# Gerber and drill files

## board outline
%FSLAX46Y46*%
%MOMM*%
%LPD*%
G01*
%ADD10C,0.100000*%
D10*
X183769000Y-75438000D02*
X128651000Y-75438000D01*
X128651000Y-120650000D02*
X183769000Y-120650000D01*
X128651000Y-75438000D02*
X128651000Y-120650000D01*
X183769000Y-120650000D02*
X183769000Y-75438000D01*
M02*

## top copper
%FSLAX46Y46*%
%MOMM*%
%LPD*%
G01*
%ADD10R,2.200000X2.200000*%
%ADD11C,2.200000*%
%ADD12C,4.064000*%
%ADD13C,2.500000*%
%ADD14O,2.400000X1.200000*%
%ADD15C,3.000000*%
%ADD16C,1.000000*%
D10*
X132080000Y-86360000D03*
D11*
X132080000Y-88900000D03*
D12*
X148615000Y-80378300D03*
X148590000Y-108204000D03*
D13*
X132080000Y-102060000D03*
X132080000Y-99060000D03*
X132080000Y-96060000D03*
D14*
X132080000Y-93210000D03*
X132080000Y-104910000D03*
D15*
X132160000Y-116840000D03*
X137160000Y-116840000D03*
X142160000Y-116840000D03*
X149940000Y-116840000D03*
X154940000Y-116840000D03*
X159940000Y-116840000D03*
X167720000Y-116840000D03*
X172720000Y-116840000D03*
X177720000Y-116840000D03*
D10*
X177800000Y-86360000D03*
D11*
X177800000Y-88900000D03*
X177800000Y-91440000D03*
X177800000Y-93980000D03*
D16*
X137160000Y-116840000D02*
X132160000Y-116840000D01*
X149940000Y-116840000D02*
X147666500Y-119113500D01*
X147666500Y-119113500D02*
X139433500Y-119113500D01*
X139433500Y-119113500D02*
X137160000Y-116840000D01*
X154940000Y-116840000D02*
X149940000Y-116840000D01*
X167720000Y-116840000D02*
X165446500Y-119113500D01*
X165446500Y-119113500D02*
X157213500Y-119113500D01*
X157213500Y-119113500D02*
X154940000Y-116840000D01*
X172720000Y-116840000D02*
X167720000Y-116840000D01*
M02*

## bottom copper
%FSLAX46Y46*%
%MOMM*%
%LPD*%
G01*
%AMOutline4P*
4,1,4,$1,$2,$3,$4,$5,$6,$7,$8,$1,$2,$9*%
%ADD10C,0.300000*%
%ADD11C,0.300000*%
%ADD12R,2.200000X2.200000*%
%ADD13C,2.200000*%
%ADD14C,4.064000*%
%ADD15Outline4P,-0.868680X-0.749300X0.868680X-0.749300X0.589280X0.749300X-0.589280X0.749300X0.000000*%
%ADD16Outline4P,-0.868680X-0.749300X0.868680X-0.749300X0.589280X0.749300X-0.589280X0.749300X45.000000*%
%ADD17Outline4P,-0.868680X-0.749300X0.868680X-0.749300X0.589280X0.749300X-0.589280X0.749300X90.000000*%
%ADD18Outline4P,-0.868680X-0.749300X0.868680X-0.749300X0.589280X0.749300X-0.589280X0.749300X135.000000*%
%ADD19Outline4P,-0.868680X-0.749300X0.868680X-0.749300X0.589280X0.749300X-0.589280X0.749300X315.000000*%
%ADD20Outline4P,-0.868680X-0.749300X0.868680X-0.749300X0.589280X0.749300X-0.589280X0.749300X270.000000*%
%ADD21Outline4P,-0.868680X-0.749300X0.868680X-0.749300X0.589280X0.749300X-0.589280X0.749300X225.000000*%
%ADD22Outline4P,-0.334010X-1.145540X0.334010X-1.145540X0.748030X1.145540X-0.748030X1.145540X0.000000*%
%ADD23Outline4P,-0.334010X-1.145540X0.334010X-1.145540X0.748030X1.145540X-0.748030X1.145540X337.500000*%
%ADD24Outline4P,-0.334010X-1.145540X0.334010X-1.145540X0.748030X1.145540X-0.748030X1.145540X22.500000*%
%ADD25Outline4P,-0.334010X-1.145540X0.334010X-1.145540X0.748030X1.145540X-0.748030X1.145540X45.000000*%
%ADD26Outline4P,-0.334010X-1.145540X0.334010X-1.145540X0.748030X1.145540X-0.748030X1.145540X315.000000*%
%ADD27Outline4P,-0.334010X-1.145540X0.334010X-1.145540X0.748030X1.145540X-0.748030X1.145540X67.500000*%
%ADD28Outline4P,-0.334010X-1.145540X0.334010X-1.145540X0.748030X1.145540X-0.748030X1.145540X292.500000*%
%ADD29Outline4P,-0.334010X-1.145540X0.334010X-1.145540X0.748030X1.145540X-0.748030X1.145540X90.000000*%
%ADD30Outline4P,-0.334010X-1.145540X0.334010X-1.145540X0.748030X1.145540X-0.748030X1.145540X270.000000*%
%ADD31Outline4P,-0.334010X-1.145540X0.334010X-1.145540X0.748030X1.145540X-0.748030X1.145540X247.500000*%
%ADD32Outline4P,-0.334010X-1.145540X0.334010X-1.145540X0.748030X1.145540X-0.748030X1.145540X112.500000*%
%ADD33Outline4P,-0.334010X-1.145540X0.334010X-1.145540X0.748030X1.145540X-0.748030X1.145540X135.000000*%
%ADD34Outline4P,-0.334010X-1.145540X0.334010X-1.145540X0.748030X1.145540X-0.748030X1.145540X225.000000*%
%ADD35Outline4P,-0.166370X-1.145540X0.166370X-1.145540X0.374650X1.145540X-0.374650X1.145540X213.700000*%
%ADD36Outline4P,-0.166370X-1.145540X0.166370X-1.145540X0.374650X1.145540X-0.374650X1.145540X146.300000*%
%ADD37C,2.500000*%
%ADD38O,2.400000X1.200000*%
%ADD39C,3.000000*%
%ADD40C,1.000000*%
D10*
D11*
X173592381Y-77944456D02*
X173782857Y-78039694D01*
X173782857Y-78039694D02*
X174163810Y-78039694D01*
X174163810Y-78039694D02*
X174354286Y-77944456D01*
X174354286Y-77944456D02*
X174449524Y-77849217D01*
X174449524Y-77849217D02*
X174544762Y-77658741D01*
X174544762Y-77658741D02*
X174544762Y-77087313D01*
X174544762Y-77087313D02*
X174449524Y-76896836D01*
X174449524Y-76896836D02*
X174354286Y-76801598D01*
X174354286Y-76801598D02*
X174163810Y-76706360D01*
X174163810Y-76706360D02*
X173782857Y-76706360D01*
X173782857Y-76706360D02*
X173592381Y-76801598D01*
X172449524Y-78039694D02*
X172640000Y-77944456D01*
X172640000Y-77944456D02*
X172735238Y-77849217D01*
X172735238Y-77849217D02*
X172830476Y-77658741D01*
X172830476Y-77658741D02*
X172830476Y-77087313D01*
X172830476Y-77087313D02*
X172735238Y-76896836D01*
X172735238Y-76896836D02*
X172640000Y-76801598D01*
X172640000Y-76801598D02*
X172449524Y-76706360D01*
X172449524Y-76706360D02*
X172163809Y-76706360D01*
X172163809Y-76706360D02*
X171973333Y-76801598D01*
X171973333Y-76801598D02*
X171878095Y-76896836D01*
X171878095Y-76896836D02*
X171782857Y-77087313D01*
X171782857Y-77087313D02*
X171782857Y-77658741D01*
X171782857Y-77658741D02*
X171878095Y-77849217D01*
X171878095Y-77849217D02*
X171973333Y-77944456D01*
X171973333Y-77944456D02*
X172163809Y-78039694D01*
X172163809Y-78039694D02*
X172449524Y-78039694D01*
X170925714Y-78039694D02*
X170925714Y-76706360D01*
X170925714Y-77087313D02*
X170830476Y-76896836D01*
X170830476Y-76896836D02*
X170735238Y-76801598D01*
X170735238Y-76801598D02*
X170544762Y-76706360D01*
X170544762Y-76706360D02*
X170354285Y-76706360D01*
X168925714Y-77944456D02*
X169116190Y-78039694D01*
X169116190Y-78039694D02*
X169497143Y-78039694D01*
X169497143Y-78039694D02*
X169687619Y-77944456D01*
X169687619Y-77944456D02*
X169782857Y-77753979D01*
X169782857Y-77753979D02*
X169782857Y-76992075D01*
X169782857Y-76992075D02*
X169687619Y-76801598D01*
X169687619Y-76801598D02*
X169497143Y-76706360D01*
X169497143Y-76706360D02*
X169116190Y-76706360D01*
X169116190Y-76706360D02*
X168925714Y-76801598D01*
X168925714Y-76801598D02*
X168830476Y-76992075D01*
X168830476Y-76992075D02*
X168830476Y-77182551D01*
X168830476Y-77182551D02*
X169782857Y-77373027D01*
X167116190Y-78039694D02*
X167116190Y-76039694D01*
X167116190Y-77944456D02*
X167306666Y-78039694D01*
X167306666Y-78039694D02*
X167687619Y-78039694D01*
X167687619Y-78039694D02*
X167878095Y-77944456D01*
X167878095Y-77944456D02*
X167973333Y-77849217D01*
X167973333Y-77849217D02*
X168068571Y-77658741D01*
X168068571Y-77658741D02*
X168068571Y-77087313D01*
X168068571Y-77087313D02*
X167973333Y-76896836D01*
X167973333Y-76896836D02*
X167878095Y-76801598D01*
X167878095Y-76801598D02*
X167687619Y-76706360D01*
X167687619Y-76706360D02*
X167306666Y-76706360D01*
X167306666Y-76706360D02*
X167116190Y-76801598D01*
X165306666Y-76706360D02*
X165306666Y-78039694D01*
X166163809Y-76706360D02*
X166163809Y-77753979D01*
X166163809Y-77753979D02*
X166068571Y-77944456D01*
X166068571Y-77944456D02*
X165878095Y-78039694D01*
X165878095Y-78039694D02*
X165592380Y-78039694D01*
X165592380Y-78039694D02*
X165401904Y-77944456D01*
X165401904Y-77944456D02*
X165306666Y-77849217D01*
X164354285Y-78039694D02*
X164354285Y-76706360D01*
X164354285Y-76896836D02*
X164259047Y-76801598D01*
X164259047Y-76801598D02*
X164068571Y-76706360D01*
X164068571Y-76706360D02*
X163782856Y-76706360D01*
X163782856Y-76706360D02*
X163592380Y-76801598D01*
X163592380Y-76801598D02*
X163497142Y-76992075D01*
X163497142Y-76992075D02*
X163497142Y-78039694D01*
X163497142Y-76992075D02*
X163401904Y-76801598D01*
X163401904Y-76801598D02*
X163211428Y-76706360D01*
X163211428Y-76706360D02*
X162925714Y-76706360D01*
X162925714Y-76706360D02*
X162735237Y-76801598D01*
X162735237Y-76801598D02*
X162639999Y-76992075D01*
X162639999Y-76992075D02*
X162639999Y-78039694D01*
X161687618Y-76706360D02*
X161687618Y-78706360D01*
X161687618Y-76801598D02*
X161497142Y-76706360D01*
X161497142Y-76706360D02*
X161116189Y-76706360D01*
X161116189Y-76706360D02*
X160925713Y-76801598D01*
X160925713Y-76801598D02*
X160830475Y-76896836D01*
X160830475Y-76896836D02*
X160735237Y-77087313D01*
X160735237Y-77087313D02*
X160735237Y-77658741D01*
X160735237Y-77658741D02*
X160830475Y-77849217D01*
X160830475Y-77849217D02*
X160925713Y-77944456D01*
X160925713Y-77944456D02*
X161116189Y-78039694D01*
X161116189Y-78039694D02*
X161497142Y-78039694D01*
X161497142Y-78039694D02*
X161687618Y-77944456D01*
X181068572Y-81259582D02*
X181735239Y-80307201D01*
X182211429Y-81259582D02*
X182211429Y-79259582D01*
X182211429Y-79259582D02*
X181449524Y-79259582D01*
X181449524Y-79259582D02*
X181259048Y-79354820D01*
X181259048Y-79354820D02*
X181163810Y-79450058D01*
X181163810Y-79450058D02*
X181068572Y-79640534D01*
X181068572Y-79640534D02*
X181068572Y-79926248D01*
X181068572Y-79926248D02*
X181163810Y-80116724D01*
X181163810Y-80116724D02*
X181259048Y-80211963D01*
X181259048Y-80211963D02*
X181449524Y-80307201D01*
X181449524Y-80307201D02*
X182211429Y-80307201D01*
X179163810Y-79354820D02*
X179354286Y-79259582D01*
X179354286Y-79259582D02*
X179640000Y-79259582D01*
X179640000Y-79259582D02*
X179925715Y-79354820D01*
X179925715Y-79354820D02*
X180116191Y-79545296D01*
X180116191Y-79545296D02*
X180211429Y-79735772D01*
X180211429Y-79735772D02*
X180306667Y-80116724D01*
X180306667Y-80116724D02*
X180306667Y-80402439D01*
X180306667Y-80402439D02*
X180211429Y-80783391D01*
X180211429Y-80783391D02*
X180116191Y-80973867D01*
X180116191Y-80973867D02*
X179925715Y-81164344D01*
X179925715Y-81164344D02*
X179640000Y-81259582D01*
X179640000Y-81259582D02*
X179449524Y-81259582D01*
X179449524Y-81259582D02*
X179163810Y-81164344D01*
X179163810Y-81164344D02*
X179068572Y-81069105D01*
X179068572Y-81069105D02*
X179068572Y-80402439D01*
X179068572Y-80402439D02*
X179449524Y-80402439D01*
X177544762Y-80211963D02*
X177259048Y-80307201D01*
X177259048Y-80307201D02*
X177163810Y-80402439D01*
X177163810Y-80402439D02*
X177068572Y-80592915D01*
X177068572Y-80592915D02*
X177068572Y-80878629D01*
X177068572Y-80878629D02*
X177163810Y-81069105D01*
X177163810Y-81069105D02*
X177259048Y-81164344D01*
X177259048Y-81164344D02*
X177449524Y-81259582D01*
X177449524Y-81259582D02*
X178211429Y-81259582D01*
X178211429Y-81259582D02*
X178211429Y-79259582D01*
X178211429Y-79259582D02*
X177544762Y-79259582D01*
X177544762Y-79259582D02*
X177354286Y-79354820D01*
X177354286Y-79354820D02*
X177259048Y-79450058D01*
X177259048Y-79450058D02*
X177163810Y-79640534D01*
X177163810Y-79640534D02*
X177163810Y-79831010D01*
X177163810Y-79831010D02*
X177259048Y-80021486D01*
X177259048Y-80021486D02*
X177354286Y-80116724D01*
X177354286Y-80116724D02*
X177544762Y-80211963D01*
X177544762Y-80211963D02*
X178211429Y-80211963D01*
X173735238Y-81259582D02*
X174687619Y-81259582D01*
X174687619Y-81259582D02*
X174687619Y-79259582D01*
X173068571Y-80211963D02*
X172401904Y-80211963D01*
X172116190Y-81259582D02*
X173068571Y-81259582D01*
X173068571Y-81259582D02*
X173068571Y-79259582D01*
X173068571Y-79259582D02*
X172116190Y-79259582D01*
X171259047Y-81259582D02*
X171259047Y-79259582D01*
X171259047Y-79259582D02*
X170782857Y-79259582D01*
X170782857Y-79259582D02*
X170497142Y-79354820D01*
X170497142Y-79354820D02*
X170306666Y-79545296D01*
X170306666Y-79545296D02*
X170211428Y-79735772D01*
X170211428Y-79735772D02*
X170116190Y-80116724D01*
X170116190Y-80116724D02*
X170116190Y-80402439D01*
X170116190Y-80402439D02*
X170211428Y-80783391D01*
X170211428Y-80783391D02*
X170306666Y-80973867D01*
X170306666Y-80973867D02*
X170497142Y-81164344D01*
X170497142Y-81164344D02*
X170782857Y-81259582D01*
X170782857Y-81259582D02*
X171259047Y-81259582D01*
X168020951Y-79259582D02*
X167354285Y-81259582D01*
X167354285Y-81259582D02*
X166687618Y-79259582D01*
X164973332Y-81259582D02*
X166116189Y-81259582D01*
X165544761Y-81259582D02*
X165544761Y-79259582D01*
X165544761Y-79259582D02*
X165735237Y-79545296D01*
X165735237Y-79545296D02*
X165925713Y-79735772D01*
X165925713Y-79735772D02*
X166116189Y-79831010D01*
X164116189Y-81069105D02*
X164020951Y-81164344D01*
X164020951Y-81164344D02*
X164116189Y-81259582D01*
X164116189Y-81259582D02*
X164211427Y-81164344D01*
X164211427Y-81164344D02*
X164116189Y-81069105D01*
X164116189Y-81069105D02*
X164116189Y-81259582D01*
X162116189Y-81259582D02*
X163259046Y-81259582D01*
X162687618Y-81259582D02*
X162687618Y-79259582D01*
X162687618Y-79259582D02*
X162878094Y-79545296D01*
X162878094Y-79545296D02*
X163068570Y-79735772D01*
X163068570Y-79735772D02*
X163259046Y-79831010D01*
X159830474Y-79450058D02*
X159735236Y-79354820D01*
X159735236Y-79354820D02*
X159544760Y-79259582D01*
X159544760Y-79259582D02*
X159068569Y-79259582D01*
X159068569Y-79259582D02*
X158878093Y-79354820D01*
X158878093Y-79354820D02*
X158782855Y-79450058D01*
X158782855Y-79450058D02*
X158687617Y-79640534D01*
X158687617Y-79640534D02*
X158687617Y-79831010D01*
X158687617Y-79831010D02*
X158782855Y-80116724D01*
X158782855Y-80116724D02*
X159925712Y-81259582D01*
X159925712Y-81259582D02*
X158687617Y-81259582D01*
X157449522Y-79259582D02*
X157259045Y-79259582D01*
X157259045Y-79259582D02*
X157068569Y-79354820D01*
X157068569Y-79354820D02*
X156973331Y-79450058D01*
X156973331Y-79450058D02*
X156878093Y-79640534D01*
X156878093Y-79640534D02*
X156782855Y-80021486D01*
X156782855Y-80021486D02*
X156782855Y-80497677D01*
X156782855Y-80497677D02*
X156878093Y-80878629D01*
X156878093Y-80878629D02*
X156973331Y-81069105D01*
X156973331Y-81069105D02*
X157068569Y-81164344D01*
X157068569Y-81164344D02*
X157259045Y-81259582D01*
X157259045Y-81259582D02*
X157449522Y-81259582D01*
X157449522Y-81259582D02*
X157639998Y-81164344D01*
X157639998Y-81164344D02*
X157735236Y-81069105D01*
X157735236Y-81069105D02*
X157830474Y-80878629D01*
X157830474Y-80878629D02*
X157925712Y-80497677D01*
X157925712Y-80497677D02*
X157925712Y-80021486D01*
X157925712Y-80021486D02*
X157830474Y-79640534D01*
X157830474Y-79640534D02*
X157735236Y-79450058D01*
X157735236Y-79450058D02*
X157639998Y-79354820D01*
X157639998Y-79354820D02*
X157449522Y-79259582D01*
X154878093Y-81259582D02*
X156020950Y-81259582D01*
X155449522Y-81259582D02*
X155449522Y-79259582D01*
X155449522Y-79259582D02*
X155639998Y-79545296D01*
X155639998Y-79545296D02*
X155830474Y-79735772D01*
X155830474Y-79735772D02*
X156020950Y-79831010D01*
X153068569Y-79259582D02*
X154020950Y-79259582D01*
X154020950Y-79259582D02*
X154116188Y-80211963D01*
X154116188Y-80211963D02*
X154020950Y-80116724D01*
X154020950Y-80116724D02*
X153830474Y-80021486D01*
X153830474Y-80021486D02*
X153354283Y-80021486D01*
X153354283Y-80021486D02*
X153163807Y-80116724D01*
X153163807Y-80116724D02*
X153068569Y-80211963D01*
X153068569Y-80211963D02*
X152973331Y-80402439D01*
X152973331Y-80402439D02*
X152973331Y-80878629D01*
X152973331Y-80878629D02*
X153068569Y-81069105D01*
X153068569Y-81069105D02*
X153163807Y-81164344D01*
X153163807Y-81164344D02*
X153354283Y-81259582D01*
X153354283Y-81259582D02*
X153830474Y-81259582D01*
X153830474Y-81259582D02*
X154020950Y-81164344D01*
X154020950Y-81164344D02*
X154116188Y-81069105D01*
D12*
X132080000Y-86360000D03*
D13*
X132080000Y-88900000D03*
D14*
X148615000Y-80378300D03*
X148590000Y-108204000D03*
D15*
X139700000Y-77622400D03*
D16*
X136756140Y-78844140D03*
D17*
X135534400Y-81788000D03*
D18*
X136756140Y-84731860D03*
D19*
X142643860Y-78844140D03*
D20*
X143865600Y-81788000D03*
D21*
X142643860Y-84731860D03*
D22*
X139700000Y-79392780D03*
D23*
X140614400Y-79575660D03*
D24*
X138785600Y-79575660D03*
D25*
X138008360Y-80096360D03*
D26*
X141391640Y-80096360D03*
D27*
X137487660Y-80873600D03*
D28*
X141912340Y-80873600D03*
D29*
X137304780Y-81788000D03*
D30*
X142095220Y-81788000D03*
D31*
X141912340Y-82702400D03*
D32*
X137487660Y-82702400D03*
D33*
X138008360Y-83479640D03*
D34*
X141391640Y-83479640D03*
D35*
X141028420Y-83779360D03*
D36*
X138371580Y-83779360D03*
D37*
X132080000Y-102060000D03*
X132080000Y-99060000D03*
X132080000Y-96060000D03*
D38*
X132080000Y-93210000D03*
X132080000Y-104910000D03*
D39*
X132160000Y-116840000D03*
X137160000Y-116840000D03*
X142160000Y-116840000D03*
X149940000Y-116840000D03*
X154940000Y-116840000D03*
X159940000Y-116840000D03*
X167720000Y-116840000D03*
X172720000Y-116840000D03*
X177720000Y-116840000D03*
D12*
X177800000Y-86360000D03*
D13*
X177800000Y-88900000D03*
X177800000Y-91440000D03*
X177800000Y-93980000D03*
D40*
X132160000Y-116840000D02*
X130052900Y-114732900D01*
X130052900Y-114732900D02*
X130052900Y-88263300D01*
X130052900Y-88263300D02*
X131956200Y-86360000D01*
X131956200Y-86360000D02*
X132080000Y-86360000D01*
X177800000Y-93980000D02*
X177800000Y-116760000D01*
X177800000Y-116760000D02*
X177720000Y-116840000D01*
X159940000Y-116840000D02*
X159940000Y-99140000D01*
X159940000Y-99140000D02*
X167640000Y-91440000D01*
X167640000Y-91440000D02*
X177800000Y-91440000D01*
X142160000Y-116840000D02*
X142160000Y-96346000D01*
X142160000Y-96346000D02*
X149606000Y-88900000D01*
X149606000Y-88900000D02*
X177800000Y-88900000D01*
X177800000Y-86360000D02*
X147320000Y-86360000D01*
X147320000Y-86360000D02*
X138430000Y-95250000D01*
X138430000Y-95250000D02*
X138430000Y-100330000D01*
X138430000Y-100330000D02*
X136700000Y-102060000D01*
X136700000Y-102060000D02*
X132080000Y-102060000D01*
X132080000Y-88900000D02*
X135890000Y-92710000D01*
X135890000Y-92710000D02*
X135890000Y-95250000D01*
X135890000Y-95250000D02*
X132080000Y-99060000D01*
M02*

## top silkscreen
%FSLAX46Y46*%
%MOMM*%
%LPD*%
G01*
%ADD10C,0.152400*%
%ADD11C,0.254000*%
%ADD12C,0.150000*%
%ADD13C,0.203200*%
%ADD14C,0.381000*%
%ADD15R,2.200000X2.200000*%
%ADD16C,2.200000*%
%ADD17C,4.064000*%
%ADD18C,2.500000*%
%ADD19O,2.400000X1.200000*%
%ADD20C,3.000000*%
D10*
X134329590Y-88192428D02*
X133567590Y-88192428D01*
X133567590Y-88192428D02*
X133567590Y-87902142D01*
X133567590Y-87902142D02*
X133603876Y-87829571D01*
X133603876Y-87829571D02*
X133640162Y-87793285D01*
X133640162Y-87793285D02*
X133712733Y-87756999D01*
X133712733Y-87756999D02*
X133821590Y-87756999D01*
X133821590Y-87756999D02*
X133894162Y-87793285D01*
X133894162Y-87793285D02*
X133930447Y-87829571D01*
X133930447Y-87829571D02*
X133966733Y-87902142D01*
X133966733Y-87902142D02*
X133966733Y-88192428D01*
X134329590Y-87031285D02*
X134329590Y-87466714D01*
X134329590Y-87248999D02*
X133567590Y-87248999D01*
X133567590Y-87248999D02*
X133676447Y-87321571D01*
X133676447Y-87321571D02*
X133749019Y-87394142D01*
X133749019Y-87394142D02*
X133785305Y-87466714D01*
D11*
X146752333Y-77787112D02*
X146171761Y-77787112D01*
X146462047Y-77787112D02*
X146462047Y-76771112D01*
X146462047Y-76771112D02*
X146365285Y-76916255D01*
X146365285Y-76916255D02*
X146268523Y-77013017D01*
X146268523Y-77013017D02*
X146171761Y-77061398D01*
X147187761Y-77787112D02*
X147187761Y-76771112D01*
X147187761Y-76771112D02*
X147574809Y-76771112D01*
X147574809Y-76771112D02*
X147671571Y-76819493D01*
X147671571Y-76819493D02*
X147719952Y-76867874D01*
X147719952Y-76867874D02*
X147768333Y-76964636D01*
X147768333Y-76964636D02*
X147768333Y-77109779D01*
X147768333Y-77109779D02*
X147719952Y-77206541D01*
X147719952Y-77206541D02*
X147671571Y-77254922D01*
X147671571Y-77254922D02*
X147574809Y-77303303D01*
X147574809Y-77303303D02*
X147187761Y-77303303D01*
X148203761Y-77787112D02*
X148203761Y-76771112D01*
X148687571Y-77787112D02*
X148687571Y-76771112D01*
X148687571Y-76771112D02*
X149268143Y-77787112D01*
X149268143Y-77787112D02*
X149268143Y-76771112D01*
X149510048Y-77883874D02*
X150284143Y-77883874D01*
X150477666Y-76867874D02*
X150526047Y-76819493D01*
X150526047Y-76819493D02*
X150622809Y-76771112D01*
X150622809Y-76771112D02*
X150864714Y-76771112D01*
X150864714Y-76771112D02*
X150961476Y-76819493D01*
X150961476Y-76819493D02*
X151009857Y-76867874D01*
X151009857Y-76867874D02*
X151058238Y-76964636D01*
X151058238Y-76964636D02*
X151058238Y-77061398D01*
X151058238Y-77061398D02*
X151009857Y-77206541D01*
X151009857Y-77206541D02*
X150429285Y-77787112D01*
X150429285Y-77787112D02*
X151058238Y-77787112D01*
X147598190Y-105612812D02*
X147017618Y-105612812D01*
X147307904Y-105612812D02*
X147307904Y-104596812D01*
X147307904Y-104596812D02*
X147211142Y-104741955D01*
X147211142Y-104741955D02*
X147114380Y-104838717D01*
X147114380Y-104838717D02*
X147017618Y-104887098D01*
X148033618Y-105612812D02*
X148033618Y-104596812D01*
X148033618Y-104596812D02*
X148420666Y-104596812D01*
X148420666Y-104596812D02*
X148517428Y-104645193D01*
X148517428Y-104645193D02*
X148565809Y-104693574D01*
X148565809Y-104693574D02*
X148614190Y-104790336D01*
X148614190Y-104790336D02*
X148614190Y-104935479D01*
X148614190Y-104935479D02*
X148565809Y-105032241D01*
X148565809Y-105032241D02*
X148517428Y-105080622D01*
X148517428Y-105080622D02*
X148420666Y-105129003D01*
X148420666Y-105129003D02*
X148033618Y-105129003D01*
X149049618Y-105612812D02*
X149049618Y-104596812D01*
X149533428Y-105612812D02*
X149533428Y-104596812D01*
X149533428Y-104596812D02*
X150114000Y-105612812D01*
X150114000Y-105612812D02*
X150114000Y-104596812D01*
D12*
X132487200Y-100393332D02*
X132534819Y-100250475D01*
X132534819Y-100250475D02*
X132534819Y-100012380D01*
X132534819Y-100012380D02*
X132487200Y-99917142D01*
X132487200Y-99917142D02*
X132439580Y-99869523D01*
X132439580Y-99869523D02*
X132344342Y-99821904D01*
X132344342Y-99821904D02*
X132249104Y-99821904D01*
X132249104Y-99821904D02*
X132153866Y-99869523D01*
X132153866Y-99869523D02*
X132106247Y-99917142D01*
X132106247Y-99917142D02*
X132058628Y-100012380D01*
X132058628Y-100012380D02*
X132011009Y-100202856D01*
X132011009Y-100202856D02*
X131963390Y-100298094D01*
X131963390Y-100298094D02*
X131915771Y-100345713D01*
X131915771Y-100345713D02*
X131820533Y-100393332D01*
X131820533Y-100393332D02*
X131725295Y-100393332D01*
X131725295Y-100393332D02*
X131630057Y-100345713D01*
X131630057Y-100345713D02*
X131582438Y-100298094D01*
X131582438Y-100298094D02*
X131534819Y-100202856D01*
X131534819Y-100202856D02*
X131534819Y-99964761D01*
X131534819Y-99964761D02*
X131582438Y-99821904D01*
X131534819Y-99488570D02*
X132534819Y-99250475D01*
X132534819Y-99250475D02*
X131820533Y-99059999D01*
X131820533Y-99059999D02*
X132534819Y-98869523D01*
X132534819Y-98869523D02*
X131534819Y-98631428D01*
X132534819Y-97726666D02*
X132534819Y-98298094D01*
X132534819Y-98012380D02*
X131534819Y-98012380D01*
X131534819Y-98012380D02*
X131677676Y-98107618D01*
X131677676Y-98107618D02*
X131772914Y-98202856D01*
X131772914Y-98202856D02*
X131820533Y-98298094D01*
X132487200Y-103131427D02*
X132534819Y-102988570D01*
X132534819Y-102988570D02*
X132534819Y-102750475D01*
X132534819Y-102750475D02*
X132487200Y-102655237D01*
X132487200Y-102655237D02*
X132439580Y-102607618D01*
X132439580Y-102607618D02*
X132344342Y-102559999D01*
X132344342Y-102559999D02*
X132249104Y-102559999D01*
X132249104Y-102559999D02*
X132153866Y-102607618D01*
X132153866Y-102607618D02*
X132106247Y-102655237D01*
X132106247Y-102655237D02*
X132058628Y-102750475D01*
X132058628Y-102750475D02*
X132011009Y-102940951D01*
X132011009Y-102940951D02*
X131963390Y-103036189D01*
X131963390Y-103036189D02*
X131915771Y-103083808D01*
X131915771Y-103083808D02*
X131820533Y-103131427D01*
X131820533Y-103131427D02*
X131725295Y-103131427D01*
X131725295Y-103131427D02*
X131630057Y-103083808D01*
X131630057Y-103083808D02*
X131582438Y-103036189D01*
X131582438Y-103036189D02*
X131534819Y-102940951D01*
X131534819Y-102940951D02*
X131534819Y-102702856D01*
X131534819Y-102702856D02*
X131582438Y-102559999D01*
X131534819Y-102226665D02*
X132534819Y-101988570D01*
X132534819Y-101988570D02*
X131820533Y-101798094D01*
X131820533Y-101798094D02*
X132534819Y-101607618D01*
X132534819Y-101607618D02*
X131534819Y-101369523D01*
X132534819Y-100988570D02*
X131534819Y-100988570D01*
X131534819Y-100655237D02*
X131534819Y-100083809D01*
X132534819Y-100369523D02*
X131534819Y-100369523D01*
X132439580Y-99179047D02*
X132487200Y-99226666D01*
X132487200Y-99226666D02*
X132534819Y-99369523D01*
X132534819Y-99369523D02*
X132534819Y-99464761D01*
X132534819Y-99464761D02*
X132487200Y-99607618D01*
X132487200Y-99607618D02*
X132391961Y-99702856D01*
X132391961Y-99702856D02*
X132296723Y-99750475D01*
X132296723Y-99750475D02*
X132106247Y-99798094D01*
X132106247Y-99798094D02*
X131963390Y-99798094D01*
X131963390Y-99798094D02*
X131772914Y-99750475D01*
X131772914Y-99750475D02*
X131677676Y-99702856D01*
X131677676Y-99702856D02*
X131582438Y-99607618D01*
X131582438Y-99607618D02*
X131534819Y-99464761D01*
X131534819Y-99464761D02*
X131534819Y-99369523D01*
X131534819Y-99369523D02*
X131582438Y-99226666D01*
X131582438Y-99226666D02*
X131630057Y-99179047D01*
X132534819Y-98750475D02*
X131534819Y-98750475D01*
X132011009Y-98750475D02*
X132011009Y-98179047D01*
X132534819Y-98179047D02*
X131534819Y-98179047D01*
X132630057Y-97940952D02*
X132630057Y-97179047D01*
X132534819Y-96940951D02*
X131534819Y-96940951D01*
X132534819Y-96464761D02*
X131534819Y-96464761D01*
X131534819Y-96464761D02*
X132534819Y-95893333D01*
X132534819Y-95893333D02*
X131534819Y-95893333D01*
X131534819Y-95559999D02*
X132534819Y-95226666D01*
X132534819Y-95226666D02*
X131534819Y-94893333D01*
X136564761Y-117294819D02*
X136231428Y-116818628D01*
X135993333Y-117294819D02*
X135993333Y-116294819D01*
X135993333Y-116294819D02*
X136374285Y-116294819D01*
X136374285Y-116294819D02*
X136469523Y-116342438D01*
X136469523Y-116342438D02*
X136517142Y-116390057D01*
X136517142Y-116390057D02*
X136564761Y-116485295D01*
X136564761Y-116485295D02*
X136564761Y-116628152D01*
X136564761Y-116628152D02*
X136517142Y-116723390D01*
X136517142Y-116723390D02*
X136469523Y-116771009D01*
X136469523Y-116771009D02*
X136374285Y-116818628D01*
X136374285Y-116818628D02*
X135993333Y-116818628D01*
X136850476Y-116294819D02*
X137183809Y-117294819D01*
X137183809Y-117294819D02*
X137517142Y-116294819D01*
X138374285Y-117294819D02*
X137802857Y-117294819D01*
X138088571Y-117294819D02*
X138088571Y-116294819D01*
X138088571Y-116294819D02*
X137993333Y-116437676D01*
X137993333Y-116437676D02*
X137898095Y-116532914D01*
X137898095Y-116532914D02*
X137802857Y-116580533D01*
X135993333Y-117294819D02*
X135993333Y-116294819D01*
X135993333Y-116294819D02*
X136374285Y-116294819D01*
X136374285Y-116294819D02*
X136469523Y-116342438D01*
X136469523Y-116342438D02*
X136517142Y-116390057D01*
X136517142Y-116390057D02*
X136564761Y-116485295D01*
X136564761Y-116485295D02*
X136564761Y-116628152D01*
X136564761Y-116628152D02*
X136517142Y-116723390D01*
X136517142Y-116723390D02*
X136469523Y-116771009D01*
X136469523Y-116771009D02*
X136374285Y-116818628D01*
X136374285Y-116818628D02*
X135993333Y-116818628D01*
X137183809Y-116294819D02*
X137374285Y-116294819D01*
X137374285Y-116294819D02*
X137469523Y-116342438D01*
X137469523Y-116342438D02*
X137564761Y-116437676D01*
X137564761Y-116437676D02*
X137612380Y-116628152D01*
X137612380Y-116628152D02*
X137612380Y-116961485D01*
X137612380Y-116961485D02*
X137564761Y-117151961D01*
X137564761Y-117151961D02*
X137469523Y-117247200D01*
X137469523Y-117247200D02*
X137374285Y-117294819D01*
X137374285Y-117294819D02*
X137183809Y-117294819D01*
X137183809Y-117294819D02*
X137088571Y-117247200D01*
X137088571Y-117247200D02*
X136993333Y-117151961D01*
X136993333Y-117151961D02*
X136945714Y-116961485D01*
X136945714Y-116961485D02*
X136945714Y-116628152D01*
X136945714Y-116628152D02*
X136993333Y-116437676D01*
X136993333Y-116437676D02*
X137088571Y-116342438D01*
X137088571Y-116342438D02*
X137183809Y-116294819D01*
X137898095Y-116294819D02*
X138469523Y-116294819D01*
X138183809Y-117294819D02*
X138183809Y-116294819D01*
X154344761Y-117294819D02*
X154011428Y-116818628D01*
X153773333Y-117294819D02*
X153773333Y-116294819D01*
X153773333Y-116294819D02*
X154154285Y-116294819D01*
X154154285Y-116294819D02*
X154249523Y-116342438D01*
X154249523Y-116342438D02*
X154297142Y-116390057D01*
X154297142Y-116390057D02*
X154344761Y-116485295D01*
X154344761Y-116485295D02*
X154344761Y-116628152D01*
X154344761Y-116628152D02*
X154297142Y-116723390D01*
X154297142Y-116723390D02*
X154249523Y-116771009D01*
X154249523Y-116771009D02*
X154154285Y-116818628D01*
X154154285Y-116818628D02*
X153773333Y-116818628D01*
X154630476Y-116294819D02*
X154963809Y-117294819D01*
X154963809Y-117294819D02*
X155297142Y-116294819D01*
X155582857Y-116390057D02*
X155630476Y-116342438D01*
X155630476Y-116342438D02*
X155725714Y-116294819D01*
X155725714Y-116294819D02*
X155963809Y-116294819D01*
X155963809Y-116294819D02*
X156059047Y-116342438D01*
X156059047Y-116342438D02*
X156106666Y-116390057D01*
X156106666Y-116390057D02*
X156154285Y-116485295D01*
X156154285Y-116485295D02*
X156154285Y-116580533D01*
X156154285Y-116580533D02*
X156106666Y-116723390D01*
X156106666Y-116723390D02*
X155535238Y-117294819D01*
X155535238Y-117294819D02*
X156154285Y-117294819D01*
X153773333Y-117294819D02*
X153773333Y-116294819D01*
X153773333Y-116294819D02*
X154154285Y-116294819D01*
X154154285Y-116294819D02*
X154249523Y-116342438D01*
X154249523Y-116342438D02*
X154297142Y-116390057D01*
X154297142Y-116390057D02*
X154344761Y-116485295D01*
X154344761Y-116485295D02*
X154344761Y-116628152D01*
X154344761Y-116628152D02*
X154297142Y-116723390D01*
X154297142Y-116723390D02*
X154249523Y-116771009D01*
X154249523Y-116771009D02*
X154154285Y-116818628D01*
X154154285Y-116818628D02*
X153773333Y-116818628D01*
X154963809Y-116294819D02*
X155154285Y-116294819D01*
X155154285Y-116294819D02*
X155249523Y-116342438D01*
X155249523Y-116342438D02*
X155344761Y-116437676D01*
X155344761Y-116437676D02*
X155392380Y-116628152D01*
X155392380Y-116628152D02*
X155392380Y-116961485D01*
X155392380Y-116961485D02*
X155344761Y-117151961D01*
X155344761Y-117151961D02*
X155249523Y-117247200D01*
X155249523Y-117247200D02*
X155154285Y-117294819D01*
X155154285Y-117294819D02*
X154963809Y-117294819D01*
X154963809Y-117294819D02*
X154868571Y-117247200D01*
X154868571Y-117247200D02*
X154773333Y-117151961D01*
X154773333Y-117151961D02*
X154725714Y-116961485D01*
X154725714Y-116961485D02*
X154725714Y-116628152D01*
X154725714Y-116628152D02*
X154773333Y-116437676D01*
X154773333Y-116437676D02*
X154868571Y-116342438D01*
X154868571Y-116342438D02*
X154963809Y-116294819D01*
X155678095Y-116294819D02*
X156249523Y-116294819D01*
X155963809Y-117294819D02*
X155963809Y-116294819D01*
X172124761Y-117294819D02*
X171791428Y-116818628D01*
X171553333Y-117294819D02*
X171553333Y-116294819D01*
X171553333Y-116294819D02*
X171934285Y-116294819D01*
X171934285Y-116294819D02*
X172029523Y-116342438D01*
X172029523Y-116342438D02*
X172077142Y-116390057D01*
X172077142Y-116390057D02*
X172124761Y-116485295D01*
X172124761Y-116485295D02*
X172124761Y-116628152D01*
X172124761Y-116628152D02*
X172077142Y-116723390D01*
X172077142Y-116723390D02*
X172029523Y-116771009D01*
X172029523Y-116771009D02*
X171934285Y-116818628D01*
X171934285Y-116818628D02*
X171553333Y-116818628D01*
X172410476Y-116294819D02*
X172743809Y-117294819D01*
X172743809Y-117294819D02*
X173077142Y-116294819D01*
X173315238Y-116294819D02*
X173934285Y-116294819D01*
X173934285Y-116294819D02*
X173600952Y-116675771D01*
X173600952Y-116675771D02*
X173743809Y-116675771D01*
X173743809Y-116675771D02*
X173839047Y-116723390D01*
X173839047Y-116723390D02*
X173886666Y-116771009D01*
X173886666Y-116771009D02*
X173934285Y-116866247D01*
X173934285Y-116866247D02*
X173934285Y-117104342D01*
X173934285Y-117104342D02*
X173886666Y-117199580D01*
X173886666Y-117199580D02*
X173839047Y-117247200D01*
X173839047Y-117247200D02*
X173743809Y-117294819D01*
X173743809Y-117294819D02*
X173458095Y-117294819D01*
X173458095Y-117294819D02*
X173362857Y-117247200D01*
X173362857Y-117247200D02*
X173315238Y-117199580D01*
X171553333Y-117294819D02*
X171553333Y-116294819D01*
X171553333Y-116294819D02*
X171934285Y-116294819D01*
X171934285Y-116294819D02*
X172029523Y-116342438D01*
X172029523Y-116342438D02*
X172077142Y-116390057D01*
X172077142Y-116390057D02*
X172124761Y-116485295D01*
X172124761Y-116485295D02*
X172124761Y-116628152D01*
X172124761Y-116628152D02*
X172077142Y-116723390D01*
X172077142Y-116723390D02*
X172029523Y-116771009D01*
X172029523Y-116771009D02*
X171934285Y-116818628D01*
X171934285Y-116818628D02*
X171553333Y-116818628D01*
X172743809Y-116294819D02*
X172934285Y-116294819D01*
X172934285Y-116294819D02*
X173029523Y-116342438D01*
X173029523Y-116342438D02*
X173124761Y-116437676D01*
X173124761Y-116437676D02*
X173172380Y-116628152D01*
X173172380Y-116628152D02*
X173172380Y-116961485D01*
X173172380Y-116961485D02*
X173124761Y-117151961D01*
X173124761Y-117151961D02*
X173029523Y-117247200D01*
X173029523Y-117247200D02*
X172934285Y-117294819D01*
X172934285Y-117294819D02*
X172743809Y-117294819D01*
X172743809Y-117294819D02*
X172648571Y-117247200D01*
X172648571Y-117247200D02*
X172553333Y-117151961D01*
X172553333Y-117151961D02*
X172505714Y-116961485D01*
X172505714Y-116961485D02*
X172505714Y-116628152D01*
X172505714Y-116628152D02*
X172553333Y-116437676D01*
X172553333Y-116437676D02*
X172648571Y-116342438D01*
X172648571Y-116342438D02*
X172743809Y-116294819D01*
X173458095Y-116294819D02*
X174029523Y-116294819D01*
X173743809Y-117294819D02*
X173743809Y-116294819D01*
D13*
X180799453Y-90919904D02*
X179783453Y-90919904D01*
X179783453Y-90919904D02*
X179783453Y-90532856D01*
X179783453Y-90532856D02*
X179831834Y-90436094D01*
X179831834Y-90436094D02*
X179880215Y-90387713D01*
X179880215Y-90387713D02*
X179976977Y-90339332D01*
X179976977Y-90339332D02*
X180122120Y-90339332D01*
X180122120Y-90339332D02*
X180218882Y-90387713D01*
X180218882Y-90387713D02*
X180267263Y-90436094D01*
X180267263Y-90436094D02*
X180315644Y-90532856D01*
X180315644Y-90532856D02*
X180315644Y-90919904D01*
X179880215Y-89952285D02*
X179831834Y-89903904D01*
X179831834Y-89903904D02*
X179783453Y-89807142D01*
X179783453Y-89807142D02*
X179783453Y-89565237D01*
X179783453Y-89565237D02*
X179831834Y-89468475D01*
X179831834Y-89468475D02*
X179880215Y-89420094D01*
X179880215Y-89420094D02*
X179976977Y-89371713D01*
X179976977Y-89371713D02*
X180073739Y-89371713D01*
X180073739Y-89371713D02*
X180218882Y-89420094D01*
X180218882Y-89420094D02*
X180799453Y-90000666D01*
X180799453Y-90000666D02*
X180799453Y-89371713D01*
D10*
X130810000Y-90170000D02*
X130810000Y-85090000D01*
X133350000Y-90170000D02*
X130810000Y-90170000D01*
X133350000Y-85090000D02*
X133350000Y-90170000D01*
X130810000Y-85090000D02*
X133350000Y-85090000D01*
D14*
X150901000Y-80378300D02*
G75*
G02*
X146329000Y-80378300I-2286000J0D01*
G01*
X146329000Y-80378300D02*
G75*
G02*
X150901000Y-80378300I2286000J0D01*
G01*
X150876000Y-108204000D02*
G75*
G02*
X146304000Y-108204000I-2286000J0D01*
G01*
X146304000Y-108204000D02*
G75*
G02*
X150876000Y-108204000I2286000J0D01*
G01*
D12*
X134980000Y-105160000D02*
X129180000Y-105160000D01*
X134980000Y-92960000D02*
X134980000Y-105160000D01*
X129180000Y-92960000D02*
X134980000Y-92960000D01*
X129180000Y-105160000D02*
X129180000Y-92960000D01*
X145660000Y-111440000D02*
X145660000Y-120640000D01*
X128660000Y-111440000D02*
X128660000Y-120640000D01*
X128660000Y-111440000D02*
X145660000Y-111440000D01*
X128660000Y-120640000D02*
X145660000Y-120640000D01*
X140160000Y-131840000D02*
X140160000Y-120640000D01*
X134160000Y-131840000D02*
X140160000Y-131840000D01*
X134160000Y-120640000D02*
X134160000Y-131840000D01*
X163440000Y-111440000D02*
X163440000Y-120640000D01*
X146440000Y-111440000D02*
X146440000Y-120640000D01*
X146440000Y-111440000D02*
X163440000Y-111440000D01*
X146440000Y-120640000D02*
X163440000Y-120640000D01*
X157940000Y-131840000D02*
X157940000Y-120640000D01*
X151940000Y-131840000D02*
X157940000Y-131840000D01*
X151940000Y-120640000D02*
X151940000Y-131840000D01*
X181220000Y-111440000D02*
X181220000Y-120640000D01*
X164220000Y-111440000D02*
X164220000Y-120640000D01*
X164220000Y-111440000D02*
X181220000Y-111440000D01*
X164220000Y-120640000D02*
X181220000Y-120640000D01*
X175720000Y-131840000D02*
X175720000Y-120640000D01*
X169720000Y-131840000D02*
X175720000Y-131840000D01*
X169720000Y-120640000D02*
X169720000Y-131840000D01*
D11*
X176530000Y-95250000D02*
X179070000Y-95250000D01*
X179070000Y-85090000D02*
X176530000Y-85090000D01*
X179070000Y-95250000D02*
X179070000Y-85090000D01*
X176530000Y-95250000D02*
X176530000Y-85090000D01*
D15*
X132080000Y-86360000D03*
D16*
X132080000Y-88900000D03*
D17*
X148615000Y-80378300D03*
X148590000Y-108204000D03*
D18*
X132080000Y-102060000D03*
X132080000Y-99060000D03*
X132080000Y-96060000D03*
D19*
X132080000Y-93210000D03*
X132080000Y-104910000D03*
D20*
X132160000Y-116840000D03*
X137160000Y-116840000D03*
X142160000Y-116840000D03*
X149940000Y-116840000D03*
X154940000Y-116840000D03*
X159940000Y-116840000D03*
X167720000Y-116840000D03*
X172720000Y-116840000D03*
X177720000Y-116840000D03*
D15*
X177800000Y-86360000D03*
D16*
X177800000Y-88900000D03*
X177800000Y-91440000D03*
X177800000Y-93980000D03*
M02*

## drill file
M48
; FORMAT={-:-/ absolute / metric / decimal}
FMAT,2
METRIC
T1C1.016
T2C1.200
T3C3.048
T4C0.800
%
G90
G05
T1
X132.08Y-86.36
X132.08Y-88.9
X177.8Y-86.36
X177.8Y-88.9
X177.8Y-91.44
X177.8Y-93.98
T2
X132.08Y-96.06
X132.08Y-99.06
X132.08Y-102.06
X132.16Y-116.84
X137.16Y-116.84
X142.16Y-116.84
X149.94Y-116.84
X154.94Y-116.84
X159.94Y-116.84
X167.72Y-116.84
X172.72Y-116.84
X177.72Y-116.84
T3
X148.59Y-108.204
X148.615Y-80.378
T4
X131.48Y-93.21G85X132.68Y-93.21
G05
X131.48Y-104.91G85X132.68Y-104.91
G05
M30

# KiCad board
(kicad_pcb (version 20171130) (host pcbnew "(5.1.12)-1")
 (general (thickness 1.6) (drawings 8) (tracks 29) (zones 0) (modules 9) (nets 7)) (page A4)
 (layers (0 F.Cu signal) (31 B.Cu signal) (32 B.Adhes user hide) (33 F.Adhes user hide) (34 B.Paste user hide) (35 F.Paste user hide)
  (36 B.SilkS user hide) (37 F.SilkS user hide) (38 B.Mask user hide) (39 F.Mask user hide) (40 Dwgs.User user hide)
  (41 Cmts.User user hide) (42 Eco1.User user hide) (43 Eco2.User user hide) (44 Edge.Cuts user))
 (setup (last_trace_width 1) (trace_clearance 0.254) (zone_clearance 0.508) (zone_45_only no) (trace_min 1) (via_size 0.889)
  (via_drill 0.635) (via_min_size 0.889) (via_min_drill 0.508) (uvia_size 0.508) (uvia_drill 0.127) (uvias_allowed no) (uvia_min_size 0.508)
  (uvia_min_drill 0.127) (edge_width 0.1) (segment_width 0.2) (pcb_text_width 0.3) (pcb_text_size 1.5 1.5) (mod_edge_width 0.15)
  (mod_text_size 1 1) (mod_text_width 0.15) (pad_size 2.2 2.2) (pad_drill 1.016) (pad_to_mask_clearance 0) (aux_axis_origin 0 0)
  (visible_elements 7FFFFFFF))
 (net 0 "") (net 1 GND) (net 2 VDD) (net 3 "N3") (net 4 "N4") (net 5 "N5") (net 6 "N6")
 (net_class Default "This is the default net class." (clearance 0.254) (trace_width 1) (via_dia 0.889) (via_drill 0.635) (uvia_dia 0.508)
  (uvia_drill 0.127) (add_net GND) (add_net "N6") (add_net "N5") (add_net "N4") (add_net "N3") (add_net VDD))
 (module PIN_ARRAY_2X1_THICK (layer F.Cu) (at 132.08 87.63 270)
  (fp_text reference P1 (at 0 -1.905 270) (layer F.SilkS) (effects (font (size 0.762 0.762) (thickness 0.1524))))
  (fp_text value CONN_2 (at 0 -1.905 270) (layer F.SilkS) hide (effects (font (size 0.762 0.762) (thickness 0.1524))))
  (fp_line (start 2.54 1.27) (end -2.54 1.27) (layer F.SilkS) (width 0.1524))
  (fp_line (start 2.54 -1.27) (end 2.54 1.27) (layer F.SilkS) (width 0.1524))
  (fp_line (start -2.54 -1.27) (end 2.54 -1.27) (layer F.SilkS) (width 0.1524))
  (fp_line (start -2.54 1.27) (end -2.54 -1.27) (layer F.SilkS) (width 0.1524))
  (pad 1 thru_hole rect (at -1.27 0 270) (size 2.2 2.2) (drill 1.016) (layers *.Cu *.Mask F.SilkS) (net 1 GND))
  (pad 2 thru_hole circle (at 1.27 0 270) (size 2.2 2.2) (drill 1.016) (layers *.Cu *.Mask F.SilkS) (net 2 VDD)))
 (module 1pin (layer F.Cu) (at 148.615 80.3783)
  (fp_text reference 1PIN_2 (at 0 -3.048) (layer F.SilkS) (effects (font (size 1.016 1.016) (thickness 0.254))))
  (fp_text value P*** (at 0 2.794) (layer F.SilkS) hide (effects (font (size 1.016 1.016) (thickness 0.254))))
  (fp_circle (center 0 0) (end 0 -2.286) (layer F.SilkS) (width 0.381))
  (pad 1 thru_hole circle (at 0 0) (size 4.064 4.064) (drill 3.048) (layers *.Cu *.Mask F.SilkS)))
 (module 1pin (layer F.Cu) (at 148.59 108.204)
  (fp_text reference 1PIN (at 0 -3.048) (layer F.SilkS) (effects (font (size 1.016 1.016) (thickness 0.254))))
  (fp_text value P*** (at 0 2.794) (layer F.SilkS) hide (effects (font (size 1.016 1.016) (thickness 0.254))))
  (fp_circle (center 0 0) (end 0 -2.286) (layer F.SilkS) (width 0.381))
  (pad 1 thru_hole circle (at 0 0) (size 4.064 4.064) (drill 3.048) (layers *.Cu *.Mask F.SilkS)))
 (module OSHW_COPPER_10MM (layer B.Cu) (at 139.7 81.788 180) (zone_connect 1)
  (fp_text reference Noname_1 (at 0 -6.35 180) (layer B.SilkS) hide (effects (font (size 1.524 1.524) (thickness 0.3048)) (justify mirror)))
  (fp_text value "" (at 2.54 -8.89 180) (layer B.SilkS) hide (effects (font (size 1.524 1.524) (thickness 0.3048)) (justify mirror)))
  (pad "" smd trapezoid (at 0 4.1656) (size 1.45796 1.4986) (rect_delta 0 0.2794) (layers B.Cu B.Paste B.Mask) (zone_connect 1))
  (pad "" smd trapezoid (at 2.94386 2.94386 45) (size 1.45796 1.4986) (rect_delta 0 0.2794) (layers B.Cu B.Paste B.Mask) (zone_connect 1))
  (pad "" smd trapezoid (at 4.1656 0 90) (size 1.45796 1.4986) (rect_delta 0 0.2794) (layers B.Cu B.Paste B.Mask) (zone_connect 1))
  (pad "" smd trapezoid (at 2.94386 -2.94386 135) (size 1.45796 1.4986) (rect_delta 0 0.2794) (layers B.Cu B.Paste B.Mask) (zone_connect 1))
  (pad "" smd trapezoid (at -2.94386 2.94386 315) (size 1.45796 1.4986) (rect_delta 0 0.2794) (layers B.Cu B.Paste B.Mask) (zone_connect 1))
  (pad "" smd trapezoid (at -4.1656 0 270) (size 1.45796 1.4986) (rect_delta 0 0.2794) (layers B.Cu B.Paste B.Mask) (zone_connect 1))
  (pad "" smd trapezoid (at -2.94386 -2.94386 225) (size 1.45796 1.4986) (rect_delta 0 0.2794) (layers B.Cu B.Paste B.Mask) (zone_connect 1))
  (pad "" smd trapezoid (at 0 2.39522) (size 1.08204 2.29108) (rect_delta 0 -0.41402) (layers B.Cu B.Paste B.Mask) (zone_connect 1))
  (pad "" smd trapezoid (at -0.9144 2.21234 337.5) (size 1.08204 2.29108) (rect_delta 0 -0.41402) (layers B.Cu B.Paste B.Mask)
   (zone_connect 1))
  (pad "" smd trapezoid (at 0.9144 2.21234 22.5) (size 1.08204 2.29108) (rect_delta 0 -0.41402) (layers B.Cu B.Paste B.Mask)
   (zone_connect 1))
  (pad "" smd trapezoid (at 1.69164 1.69164 45) (size 1.08204 2.29108) (rect_delta 0 -0.41402) (layers B.Cu B.Paste B.Mask) (zone_connect 1))
  (pad "" smd trapezoid (at -1.69164 1.69164 315) (size 1.08204 2.29108) (rect_delta 0 -0.41402) (layers B.Cu B.Paste B.Mask)
   (zone_connect 1))
  (pad "" smd trapezoid (at 2.21234 0.9144 67.5) (size 1.08204 2.29108) (rect_delta 0 -0.41402) (layers B.Cu B.Paste B.Mask)
   (zone_connect 1))
  (pad "" smd trapezoid (at -2.21234 0.9144 292.5) (size 1.08204 2.29108) (rect_delta 0 -0.41402) (layers B.Cu B.Paste B.Mask)
   (zone_connect 1))
  (pad "" smd trapezoid (at 2.39522 0 90) (size 1.08204 2.29108) (rect_delta 0 -0.41402) (layers B.Cu B.Paste B.Mask) (zone_connect 1))
  (pad "" smd trapezoid (at -2.39522 0 270) (size 1.08204 2.29108) (rect_delta 0 -0.41402) (layers B.Cu B.Paste B.Mask) (zone_connect 1))
  (pad "" smd trapezoid (at -2.21234 -0.9144 247.5) (size 1.08204 2.29108) (rect_delta 0 -0.41402) (layers B.Cu B.Paste B.Mask)
   (zone_connect 1))
  (pad "" smd trapezoid (at 2.21234 -0.9144 112.5) (size 1.08204 2.29108) (rect_delta 0 -0.41402) (layers B.Cu B.Paste B.Mask)
   (zone_connect 1))
  (pad "" smd trapezoid (at 1.69164 -1.69164 135) (size 1.08204 2.29108) (rect_delta 0 -0.41402) (layers B.Cu B.Paste B.Mask)
   (zone_connect 1))
  (pad "" smd trapezoid (at -1.69164 -1.69164 225) (size 1.08204 2.29108) (rect_delta 0 -0.41402) (layers B.Cu B.Paste B.Mask)
   (zone_connect 1))
  (pad "" smd trapezoid (at -1.32842 -1.99136 213.7) (size 0.54102 2.29108) (rect_delta 0 -0.20828) (layers B.Cu B.Paste B.Mask)
   (zone_connect 1))
  (pad "" smd trapezoid (at 1.32842 -1.99136 146.3) (size 0.54102 2.29108) (rect_delta 0 -0.20828) (layers B.Cu B.Paste B.Mask)
   (zone_connect 1)))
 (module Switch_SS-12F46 (layer F.Cu) (at 132.08 99.06 90)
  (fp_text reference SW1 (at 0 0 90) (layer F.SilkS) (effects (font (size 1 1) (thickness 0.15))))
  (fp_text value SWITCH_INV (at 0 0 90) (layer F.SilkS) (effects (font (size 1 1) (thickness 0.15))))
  (fp_line (start -6.1 2.9) (end -6.1 -2.9) (layer F.SilkS) (width 0.15))
  (fp_line (start 6.1 2.9) (end -6.1 2.9) (layer F.SilkS) (width 0.15))
  (fp_line (start 6.1 -2.9) (end 6.1 2.9) (layer F.SilkS) (width 0.15))
  (fp_line (start -6.1 -2.9) (end 6.1 -2.9) (layer F.SilkS) (width 0.15))
  (pad 1 thru_hole circle (at -3 0 90) (size 2.5 2.5) (drill 1.2) (layers *.Cu *.Mask F.SilkS) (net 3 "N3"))
  (pad 2 thru_hole circle (at 0 0 90) (size 2.5 2.5) (drill 1.2) (layers *.Cu *.Mask F.SilkS) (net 2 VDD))
  (pad 3 thru_hole circle (at 3 0 90) (size 2.5 2.5) (drill 1.2) (layers *.Cu *.Mask F.SilkS))
  (pad "" np_thru_hole oval (at 5.85 0 90) (size 1.2 2.4) (drill oval 0.8 2) (layers *.Cu *.Mask F.SilkS))
  (pad "" np_thru_hole oval (at -5.85 0 90) (size 1.2 2.4) (drill oval 0.8 2) (layers *.Cu *.Mask F.SilkS)))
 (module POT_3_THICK (layer F.Cu) (at 137.16 116.84)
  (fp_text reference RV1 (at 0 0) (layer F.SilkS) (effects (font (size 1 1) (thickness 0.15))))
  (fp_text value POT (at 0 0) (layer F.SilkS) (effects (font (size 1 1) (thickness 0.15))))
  (fp_line (start 8.5 -5.4) (end 8.5 3.8) (layer F.SilkS) (width 0.15))
  (fp_line (start -8.5 -5.4) (end -8.5 3.8) (layer F.SilkS) (width 0.15))
  (fp_line (start -8.5 -5.4) (end 8.5 -5.4) (layer F.SilkS) (width 0.15))
  (fp_line (start -8.5 3.8) (end 8.5 3.8) (layer F.SilkS) (width 0.15))
  (fp_line (start 3 15) (end 3 3.8) (layer F.SilkS) (width 0.15))
  (fp_line (start -3 15) (end 3 15) (layer F.SilkS) (width 0.15))
  (fp_line (start -3 3.8) (end -3 15) (layer F.SilkS) (width 0.15))
  (pad 1 thru_hole circle (at -5 0) (size 3 3) (drill 1.2) (layers *.Cu *.Mask F.SilkS) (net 1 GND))
  (pad 2 thru_hole circle (at 0 0) (size 3 3) (drill 1.2) (layers *.Cu *.Mask F.SilkS) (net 1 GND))
  (pad 3 thru_hole circle (at 5 0) (size 3 3) (drill 1.2) (layers *.Cu *.Mask F.SilkS) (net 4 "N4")))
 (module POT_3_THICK (layer F.Cu) (at 154.94 116.84)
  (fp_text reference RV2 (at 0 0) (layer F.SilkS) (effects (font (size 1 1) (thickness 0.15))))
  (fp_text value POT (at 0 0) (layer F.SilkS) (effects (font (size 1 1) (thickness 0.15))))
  (fp_line (start 8.5 -5.4) (end 8.5 3.8) (layer F.SilkS) (width 0.15))
  (fp_line (start -8.5 -5.4) (end -8.5 3.8) (layer F.SilkS) (width 0.15))
  (fp_line (start -8.5 -5.4) (end 8.5 -5.4) (layer F.SilkS) (width 0.15))
  (fp_line (start -8.5 3.8) (end 8.5 3.8) (layer F.SilkS) (width 0.15))
  (fp_line (start 3 15) (end 3 3.8) (layer F.SilkS) (width 0.15))
  (fp_line (start -3 15) (end 3 15) (layer F.SilkS) (width 0.15))
  (fp_line (start -3 3.8) (end -3 15) (layer F.SilkS) (width 0.15))
  (pad 1 thru_hole circle (at -5 0) (size 3 3) (drill 1.2) (layers *.Cu *.Mask F.SilkS) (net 1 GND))
  (pad 2 thru_hole circle (at 0 0) (size 3 3) (drill 1.2) (layers *.Cu *.Mask F.SilkS) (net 1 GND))
  (pad 3 thru_hole circle (at 5 0) (size 3 3) (drill 1.2) (layers *.Cu *.Mask F.SilkS) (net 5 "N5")))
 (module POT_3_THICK (layer F.Cu) (at 172.72 116.84)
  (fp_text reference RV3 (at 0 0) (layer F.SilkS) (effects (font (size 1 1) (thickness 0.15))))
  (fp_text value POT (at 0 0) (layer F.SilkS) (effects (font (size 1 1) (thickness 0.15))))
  (fp_line (start 8.5 -5.4) (end 8.5 3.8) (layer F.SilkS) (width 0.15))
  (fp_line (start -8.5 -5.4) (end -8.5 3.8) (layer F.SilkS) (width 0.15))
  (fp_line (start -8.5 -5.4) (end 8.5 -5.4) (layer F.SilkS) (width 0.15))
  (fp_line (start -8.5 3.8) (end 8.5 3.8) (layer F.SilkS) (width 0.15))
  (fp_line (start 3 15) (end 3 3.8) (layer F.SilkS) (width 0.15))
  (fp_line (start -3 15) (end 3 15) (layer F.SilkS) (width 0.15))
  (fp_line (start -3 3.8) (end -3 15) (layer F.SilkS) (width 0.15))
  (pad 1 thru_hole circle (at -5 0) (size 3 3) (drill 1.2) (layers *.Cu *.Mask F.SilkS) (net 1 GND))
  (pad 2 thru_hole circle (at 0 0) (size 3 3) (drill 1.2) (layers *.Cu *.Mask F.SilkS) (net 1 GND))
  (pad 3 thru_hole circle (at 5 0) (size 3 3) (drill 1.2) (layers *.Cu *.Mask F.SilkS) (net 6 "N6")))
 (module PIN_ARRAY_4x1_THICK (layer F.Cu) (at 177.8 90.17 270)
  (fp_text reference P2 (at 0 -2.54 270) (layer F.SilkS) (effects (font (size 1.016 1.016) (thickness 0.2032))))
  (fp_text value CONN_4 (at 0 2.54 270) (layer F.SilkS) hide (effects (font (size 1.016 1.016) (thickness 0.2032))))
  (fp_line (start 5.08 1.27) (end 5.08 -1.27) (layer F.SilkS) (width 0.254))
  (fp_line (start -5.08 -1.27) (end -5.08 1.27) (layer F.SilkS) (width 0.254))
  (fp_line (start 5.08 -1.27) (end -5.08 -1.27) (layer F.SilkS) (width 0.254))
  (fp_line (start 5.08 1.27) (end -5.08 1.27) (layer F.SilkS) (width 0.254))
  (pad 1 thru_hole rect (at -3.81 0 270) (size 2.2 2.2) (drill 1.016) (layers *.Cu *.Mask F.SilkS) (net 3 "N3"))
  (pad 2 thru_hole circle (at -1.27 0 270) (size 2.2 2.2) (drill 1.016) (layers *.Cu *.Mask F.SilkS) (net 4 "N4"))
  (pad 3 thru_hole circle (at 1.27 0 270) (size 2.2 2.2) (drill 1.016) (layers *.Cu *.Mask F.SilkS) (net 5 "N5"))
  (pad 4 thru_hole circle (at 3.81 0 270) (size 2.2 2.2) (drill 1.016) (layers *.Cu *.Mask F.SilkS) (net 6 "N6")))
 (gr_line (start 183.769 75.438) (end 128.651 75.438) (angle 90) (layer Edge.Cuts) (width 0.1))
 (gr_line (start 128.651 120.65) (end 183.769 120.65) (angle 90) (layer Edge.Cuts) (width 0.1))
 (gr_line (start 128.651 75.438) (end 128.651 120.65) (angle 90) (layer Edge.Cuts) (width 0.1))
 (gr_line (start 183.769 120.65) (end 183.769 75.438) (angle 90) (layer Edge.Cuts) (width 0.1))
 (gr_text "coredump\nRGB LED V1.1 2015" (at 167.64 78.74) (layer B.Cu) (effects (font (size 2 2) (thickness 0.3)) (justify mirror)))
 (segment (start 132.16 116.84) (end 130.0529 114.7329) (width 1) (layer B.Cu) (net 1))
 (segment (start 130.0529 114.7329) (end 130.0529 88.2633) (width 1) (layer B.Cu) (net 1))
 (segment (start 130.0529 88.2633) (end 131.9562 86.36) (width 1) (layer B.Cu) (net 1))
 (segment (start 131.9562 86.36) (end 132.08 86.36) (width 1) (layer B.Cu) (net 1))
 (segment (start 137.16 116.84) (end 132.16 116.84) (width 1) (layer F.Cu) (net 1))
 (segment (start 149.94 116.84) (end 147.6665 119.1135) (width 1) (layer F.Cu) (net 1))
 (segment (start 147.6665 119.1135) (end 139.4335 119.1135) (width 1) (layer F.Cu) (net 1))
 (segment (start 139.4335 119.1135) (end 137.16 116.84) (width 1) (layer F.Cu) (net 1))
 (segment (start 154.94 116.84) (end 149.94 116.84) (width 1) (layer F.Cu) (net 1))
 (segment (start 167.72 116.84) (end 165.4465 119.1135) (width 1) (layer F.Cu) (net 1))
 (segment (start 165.4465 119.1135) (end 157.2135 119.1135) (width 1) (layer F.Cu) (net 1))
 (segment (start 157.2135 119.1135) (end 154.94 116.84) (width 1) (layer F.Cu) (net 1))
 (segment (start 172.72 116.84) (end 167.72 116.84) (width 1) (layer F.Cu) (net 1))
 (segment (start 177.8 93.98) (end 177.8 116.76) (width 1) (layer B.Cu) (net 6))
 (segment (start 177.8 116.76) (end 177.72 116.84) (width 1) (layer B.Cu) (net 6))
 (segment (start 159.94 116.84) (end 159.94 99.14) (width 1) (layer B.Cu) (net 5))
 (segment (start 159.94 99.14) (end 167.64 91.44) (width 1) (layer B.Cu) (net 5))
 (segment (start 167.64 91.44) (end 177.8 91.44) (width 1) (layer B.Cu) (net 5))
 (segment (start 142.16 116.84) (end 142.16 96.346) (width 1) (layer B.Cu) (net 4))
 (segment (start 142.16 96.346) (end 149.606 88.9) (width 1) (layer B.Cu) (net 4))
 (segment (start 149.606 88.9) (end 177.8 88.9) (width 1) (layer B.Cu) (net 4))
 (segment (start 177.8 86.36) (end 147.32 86.36) (width 1) (layer B.Cu) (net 3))
 (segment (start 147.32 86.36) (end 138.43 95.25) (width 1) (layer B.Cu) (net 3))
 (segment (start 138.43 95.25) (end 138.43 100.33) (width 1) (layer B.Cu) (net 3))
 (segment (start 138.43 100.33) (end 136.7 102.06) (width 1) (layer B.Cu) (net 3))
 (segment (start 136.7 102.06) (end 132.08 102.06) (width 1) (layer B.Cu) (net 3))
 (segment (start 132.08 88.9) (end 135.89 92.71) (width 1) (layer B.Cu) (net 2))
 (segment (start 135.89 92.71) (end 135.89 95.25) (width 1) (layer B.Cu) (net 2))
 (segment (start 135.89 95.25) (end 132.08 99.06) (width 1) (layer B.Cu) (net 2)))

